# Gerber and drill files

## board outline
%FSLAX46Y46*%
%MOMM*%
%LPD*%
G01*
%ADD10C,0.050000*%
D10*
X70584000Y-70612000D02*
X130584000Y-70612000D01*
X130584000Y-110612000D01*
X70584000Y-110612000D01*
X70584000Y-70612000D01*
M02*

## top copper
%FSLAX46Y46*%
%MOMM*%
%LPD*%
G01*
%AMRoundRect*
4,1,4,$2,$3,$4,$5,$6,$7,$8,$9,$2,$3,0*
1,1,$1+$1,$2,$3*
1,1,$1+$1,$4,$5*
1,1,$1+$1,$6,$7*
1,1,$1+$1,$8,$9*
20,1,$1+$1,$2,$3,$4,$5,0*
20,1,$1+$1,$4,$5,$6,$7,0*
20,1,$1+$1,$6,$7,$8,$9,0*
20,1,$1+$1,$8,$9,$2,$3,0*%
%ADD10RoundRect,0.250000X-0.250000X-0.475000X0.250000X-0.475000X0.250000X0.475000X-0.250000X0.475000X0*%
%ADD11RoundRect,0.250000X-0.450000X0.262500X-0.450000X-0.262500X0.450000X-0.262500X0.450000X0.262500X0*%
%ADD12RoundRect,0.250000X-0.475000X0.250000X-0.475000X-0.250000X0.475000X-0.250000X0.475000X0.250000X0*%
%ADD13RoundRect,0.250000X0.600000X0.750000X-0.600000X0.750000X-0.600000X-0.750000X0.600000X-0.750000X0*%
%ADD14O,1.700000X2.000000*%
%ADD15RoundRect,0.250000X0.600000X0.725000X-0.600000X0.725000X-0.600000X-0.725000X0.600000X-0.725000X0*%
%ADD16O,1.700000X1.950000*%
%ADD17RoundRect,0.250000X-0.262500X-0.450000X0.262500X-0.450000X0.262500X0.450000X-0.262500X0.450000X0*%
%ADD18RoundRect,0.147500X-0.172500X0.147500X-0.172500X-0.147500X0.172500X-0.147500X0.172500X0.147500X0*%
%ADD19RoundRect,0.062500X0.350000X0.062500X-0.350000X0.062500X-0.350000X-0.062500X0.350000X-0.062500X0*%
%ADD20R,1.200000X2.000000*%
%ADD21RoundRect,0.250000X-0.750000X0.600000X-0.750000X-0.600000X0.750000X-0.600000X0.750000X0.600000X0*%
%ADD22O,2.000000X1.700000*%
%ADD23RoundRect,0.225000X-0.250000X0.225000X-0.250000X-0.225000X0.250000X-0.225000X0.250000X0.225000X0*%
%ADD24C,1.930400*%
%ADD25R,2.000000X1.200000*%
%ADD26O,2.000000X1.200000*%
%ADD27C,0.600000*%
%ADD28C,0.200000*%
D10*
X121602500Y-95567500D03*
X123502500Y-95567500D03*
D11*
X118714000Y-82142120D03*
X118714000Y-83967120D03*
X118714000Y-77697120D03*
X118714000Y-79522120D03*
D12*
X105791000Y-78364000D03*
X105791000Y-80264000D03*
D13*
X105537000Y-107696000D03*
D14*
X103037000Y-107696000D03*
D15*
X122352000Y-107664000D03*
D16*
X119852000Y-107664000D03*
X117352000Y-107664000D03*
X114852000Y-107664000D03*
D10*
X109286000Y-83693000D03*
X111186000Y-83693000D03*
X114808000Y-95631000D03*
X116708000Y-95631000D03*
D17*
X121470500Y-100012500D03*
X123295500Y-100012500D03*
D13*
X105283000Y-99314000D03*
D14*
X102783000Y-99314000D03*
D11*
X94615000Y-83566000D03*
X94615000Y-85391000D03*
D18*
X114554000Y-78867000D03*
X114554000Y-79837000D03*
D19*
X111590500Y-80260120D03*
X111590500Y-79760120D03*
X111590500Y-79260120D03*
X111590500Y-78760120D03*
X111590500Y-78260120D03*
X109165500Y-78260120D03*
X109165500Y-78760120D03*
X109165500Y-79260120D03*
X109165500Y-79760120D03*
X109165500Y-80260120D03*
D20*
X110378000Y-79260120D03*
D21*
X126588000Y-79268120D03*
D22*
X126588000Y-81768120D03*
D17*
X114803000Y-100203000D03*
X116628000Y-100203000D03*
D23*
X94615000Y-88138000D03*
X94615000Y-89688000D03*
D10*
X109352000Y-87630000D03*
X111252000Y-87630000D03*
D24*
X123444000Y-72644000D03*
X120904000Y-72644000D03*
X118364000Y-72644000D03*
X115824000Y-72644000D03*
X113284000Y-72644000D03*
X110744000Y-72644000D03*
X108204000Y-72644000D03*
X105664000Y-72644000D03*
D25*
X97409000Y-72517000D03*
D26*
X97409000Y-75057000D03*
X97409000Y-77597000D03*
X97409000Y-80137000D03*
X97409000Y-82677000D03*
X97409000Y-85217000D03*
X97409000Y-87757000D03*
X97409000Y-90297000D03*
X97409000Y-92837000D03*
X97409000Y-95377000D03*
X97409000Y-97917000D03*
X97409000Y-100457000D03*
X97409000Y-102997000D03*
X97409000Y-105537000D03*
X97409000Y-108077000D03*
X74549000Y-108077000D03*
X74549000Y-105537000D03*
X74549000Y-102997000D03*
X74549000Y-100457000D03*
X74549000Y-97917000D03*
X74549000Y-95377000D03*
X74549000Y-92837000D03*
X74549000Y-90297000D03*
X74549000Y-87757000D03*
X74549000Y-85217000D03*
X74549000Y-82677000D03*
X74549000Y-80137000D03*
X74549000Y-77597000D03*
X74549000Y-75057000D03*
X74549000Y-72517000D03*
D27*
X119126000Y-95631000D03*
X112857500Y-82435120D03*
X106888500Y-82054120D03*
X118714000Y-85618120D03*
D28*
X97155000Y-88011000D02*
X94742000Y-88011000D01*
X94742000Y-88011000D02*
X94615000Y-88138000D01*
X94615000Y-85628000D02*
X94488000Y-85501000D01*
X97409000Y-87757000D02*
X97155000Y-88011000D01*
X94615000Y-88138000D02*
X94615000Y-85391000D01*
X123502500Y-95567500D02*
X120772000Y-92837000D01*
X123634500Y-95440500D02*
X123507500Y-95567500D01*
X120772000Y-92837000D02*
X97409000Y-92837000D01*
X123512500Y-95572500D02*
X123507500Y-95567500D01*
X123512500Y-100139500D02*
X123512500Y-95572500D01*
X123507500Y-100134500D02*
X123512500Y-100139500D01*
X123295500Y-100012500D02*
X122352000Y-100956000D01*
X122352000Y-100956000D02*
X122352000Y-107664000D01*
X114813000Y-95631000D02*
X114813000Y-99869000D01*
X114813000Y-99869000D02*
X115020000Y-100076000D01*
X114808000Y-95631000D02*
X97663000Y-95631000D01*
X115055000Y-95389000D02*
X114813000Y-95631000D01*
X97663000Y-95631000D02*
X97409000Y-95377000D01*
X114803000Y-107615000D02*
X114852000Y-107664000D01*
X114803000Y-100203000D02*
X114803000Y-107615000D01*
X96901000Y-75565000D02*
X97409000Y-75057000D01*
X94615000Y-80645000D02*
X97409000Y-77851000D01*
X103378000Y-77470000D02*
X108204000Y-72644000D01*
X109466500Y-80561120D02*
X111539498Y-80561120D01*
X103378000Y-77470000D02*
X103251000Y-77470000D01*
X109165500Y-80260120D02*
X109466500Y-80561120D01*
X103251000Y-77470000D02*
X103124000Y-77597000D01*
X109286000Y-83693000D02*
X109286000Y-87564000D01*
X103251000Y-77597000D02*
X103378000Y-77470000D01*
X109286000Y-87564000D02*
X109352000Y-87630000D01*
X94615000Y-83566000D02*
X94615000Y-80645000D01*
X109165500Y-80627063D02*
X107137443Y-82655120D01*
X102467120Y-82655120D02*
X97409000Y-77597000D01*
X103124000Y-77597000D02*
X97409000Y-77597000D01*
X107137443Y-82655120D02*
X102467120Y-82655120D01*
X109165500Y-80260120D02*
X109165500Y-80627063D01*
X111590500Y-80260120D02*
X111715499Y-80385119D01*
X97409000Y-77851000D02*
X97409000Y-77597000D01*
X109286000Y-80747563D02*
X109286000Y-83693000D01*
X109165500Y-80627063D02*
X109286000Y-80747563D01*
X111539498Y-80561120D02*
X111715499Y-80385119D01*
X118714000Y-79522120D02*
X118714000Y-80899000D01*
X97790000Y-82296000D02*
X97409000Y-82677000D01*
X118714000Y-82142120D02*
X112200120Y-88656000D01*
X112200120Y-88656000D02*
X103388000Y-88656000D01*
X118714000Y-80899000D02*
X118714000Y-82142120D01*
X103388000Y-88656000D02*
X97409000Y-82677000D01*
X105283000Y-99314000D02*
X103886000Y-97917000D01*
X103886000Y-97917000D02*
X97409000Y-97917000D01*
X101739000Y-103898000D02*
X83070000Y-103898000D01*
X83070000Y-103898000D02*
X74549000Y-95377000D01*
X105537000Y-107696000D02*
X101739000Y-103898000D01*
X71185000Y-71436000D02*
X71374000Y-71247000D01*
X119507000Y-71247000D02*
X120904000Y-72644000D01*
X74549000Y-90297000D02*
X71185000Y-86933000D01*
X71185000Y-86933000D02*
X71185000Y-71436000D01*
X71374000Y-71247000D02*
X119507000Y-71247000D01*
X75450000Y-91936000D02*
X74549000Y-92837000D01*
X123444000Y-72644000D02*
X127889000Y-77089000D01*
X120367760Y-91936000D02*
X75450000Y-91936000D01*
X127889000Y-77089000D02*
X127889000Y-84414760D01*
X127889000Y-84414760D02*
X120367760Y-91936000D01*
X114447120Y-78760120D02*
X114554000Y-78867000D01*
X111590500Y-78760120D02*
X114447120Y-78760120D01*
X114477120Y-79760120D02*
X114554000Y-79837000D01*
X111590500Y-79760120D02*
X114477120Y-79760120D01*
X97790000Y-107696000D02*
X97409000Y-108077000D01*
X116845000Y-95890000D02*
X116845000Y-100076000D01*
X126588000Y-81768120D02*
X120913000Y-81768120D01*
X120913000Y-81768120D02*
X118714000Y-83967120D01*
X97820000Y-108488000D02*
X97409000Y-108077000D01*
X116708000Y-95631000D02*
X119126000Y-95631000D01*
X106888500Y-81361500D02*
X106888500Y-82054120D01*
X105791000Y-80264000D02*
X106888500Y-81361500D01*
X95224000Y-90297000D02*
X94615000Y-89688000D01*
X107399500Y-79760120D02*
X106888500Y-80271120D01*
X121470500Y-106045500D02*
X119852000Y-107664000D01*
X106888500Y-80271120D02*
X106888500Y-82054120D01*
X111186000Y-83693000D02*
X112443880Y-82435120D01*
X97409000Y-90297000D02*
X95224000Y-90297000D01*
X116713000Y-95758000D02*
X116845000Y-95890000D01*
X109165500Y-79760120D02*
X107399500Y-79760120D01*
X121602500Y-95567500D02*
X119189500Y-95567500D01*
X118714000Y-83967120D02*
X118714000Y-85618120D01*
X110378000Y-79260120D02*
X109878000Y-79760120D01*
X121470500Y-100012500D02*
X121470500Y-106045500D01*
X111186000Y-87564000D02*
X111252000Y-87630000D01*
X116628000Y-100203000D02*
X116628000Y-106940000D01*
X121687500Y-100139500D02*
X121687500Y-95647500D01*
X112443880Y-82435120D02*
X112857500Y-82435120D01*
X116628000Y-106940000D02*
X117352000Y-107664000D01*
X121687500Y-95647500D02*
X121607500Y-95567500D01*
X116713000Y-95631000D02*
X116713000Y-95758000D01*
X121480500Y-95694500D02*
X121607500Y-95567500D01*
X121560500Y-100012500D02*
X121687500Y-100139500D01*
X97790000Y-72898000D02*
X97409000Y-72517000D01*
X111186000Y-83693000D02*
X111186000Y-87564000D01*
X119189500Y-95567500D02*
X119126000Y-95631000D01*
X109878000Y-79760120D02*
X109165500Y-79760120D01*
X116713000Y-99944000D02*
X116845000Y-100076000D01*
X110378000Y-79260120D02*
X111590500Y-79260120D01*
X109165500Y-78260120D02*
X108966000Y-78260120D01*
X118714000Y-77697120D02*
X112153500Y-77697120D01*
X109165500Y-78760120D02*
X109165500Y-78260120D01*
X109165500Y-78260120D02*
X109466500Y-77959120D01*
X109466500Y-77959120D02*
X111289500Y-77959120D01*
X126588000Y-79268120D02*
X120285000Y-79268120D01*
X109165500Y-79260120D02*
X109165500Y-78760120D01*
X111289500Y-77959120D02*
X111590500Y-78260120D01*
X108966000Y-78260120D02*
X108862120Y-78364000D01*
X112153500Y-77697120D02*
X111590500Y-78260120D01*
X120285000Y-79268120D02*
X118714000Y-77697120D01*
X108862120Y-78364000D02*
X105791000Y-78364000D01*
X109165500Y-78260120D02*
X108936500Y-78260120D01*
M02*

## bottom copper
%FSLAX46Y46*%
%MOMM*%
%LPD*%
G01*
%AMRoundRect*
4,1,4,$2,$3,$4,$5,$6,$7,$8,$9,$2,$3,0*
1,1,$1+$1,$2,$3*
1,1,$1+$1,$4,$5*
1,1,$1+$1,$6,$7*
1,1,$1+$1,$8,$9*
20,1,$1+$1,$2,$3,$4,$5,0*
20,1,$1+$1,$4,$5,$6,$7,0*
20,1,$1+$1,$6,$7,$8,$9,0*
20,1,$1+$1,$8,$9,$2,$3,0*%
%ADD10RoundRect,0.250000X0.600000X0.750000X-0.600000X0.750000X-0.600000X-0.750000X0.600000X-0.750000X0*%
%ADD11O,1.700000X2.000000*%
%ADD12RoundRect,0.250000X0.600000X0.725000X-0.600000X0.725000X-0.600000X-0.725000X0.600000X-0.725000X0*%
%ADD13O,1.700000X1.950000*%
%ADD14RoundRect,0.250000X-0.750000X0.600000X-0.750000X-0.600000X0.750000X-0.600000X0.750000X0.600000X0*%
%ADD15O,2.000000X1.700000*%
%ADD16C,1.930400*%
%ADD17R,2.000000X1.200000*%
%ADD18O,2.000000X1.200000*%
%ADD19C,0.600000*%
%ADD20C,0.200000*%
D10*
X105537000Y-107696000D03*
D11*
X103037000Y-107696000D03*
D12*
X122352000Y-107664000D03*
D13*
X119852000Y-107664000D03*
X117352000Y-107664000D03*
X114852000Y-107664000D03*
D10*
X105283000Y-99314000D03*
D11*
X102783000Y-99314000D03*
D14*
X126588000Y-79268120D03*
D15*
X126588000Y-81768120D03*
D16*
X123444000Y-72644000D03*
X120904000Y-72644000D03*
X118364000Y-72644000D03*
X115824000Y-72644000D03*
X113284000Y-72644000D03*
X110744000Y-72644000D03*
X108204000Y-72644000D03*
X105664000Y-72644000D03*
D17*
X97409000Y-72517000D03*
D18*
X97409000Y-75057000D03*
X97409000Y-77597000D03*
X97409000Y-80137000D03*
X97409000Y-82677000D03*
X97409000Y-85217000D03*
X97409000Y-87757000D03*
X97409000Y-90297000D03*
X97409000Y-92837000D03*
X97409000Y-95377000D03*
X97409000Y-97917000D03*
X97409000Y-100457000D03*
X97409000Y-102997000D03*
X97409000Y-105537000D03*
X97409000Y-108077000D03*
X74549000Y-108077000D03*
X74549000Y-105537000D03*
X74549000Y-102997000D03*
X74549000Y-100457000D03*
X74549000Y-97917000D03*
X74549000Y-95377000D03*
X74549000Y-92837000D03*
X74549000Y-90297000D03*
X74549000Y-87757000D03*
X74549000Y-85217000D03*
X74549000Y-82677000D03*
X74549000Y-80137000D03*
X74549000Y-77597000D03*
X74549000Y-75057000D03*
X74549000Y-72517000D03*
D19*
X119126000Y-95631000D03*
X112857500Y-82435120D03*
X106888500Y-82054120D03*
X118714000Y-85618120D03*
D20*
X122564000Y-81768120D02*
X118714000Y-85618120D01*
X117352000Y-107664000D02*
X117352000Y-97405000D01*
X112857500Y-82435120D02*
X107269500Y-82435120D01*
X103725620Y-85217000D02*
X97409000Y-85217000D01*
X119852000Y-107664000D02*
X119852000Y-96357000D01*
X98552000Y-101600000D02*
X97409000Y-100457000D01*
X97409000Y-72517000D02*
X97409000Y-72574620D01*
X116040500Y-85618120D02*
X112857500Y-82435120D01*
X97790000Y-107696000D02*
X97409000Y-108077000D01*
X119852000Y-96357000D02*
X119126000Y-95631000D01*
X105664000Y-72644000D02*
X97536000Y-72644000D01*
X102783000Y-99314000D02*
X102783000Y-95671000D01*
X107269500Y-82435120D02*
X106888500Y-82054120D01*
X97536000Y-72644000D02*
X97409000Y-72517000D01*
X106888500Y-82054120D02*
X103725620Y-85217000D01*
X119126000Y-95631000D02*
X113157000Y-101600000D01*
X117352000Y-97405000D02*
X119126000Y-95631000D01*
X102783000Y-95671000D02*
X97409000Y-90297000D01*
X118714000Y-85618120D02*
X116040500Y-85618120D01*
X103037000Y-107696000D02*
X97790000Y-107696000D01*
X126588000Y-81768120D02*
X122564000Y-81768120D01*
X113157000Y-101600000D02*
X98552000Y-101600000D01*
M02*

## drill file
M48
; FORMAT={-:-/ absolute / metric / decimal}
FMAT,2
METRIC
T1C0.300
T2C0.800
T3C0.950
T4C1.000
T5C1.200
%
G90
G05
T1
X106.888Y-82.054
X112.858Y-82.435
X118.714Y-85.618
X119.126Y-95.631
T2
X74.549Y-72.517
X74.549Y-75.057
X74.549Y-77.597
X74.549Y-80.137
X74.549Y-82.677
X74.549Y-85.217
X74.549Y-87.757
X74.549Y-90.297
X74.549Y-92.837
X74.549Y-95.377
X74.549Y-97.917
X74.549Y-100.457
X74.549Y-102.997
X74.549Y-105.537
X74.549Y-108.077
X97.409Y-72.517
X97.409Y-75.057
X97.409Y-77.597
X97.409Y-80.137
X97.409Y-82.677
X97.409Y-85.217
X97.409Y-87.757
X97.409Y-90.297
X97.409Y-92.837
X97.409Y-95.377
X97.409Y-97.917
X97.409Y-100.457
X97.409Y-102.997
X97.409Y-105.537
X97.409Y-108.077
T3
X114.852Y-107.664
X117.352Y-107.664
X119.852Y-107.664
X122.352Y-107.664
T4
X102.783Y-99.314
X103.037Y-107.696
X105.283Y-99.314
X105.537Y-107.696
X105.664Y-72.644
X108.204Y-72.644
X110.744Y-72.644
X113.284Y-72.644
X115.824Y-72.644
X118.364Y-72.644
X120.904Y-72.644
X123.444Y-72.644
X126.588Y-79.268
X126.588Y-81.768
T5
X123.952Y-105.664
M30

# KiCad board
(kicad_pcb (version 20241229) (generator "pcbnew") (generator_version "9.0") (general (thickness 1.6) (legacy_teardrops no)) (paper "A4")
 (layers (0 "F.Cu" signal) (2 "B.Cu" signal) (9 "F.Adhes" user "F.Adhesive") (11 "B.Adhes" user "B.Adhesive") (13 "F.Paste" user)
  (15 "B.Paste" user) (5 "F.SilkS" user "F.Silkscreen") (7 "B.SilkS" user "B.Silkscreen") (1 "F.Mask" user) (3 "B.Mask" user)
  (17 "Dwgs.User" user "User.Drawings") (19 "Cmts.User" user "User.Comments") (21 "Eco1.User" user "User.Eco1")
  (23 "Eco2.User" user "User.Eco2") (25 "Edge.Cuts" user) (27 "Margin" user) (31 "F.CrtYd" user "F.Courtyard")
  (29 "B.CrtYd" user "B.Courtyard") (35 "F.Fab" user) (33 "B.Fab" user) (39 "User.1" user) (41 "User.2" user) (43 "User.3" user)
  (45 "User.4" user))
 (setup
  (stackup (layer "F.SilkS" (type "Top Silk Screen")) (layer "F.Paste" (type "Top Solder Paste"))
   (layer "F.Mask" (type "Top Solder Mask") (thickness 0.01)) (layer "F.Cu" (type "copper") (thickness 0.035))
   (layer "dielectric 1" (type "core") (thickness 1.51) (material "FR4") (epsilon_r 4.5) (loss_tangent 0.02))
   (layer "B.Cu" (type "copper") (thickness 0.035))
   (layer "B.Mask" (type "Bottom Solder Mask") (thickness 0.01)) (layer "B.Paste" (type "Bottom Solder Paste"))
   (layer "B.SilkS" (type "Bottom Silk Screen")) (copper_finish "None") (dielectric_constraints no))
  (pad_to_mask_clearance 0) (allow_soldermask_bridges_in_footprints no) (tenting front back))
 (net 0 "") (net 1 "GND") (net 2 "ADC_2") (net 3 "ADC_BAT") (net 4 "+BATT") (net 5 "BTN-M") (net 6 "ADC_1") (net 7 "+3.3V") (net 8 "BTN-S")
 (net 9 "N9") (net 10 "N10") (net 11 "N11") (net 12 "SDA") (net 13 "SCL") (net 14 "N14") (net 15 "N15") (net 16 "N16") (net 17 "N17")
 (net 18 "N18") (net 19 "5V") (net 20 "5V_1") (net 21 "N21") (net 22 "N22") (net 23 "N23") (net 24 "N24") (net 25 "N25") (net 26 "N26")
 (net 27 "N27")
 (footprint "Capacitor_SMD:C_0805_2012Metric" (layer "F.Cu") (at 122.5525 95.5675)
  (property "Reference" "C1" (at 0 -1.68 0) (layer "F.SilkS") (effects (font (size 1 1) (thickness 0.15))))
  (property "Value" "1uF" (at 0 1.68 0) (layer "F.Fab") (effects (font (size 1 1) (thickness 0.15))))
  (pad "1" smd roundrect (at -0.95 0) (size 1 1.45) (layers "F.Cu" "F.Mask" "F.Paste") (roundrect_rratio 0.25) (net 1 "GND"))
  (pad "2" smd roundrect (at 0.95 0) (size 1 1.45) (layers "F.Cu" "F.Mask" "F.Paste") (roundrect_rratio 0.25) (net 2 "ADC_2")))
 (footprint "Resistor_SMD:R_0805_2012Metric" (layer "F.Cu") (at 118.714 83.05462 -90)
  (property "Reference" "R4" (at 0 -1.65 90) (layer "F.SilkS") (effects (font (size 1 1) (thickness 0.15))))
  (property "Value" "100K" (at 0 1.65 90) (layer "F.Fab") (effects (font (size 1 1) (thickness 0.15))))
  (pad "1" smd roundrect (at -0.9125 0 270) (size 1.025 1.4) (layers "F.Cu" "F.Mask" "F.Paste") (roundrect_rratio 0.243902)
   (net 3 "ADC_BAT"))
  (pad "2" smd roundrect (at 0.9125 0 270) (size 1.025 1.4) (layers "F.Cu" "F.Mask" "F.Paste") (roundrect_rratio 0.243902) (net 1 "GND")))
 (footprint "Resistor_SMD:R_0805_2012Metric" (layer "F.Cu") (at 118.714 78.60962 -90)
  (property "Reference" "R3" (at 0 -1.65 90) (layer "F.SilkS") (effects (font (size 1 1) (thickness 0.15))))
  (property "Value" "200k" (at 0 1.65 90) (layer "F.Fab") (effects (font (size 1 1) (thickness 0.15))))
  (pad "1" smd roundrect (at -0.9125 0 270) (size 1.025 1.4) (layers "F.Cu" "F.Mask" "F.Paste") (roundrect_rratio 0.243902) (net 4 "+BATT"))
  (pad "2" smd roundrect (at 0.9125 0 270) (size 1.025 1.4) (layers "F.Cu" "F.Mask" "F.Paste") (roundrect_rratio 0.243902) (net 3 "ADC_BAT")))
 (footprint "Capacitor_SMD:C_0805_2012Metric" (layer "F.Cu") (at 105.791 79.314 -90)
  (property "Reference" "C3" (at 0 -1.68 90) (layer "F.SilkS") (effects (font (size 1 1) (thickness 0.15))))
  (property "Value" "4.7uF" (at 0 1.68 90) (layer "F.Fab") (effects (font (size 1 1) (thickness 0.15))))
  (pad "1" smd roundrect (at -0.95 0 270) (size 1 1.45) (layers "F.Cu" "F.Mask" "F.Paste") (roundrect_rratio 0.25) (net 4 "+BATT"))
  (pad "2" smd roundrect (at 0.95 0 270) (size 1 1.45) (layers "F.Cu" "F.Mask" "F.Paste") (roundrect_rratio 0.25) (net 1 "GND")))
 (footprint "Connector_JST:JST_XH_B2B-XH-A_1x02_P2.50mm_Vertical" (layer "F.Cu") (at 105.537 107.696 180)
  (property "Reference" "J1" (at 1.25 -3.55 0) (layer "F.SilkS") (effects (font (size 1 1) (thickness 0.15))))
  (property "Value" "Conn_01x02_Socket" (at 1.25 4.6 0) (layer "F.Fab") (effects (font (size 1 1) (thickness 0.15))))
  (pad "1" thru_hole roundrect (at 0 0 180) (size 1.7 2) (drill 1) (layers "*.Cu" "*.Mask") (remove_unused_layers no)
   (roundrect_rratio 0.147059) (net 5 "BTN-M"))
  (pad "2" thru_hole oval (at 2.5 0 180) (size 1.7 2) (drill 1) (layers "*.Cu" "*.Mask") (remove_unused_layers no) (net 1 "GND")))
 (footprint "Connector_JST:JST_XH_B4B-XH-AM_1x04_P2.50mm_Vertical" (layer "F.Cu") (at 122.352 107.664 180)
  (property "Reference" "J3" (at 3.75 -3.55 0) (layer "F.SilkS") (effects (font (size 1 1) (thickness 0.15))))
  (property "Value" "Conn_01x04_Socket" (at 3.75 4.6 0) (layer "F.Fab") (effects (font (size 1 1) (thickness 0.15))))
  (pad "" np_thru_hole circle (at -1.6 2 180) (size 1.2 1.2) (drill 1.2) (layers "*.Cu" "*.Mask"))
  (pad "1" thru_hole roundrect (at 0 0 180) (size 1.7 1.95) (drill 0.95) (layers "*.Cu" "*.Mask") (remove_unused_layers no)
   (roundrect_rratio 0.147059) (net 2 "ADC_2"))
  (pad "2" thru_hole oval (at 2.5 0 180) (size 1.7 1.95) (drill 0.95) (layers "*.Cu" "*.Mask") (remove_unused_layers no) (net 1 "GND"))
  (pad "3" thru_hole oval (at 5 0 180) (size 1.7 1.95) (drill 0.95) (layers "*.Cu" "*.Mask") (remove_unused_layers no) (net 1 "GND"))
  (pad "4" thru_hole oval (at 7.5 0 180) (size 1.7 1.95) (drill 0.95) (layers "*.Cu" "*.Mask") (remove_unused_layers no) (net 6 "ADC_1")))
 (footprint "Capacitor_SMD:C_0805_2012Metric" (layer "F.Cu") (at 110.236 83.693)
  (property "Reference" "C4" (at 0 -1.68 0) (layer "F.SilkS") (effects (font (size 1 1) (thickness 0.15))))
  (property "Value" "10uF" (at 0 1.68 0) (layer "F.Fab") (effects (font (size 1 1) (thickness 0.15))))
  (pad "1" smd roundrect (at -0.95 0) (size 1 1.45) (layers "F.Cu" "F.Mask" "F.Paste") (roundrect_rratio 0.25) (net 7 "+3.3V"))
  (pad "2" smd roundrect (at 0.95 0) (size 1 1.45) (layers "F.Cu" "F.Mask" "F.Paste") (roundrect_rratio 0.25) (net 1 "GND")))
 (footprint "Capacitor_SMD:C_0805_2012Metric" (layer "F.Cu") (at 115.758 95.631)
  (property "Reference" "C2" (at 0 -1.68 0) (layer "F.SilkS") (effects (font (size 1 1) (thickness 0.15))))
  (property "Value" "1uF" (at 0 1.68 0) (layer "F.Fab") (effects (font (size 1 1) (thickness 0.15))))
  (pad "1" smd roundrect (at -0.95 0) (size 1 1.45) (layers "F.Cu" "F.Mask" "F.Paste") (roundrect_rratio 0.25) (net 6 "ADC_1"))
  (pad "2" smd roundrect (at 0.95 0) (size 1 1.45) (layers "F.Cu" "F.Mask" "F.Paste") (roundrect_rratio 0.25) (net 1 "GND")))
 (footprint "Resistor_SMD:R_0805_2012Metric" (layer "F.Cu") (at 122.383 100.0125)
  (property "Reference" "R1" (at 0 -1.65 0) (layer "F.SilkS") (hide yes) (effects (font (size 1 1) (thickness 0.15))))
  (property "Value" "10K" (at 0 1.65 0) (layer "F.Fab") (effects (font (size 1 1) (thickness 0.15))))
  (pad "1" smd roundrect (at -0.9125 0) (size 1.025 1.4) (layers "F.Cu" "F.Mask" "F.Paste") (roundrect_rratio 0.243902) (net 1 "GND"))
  (pad "2" smd roundrect (at 0.9125 0) (size 1.025 1.4) (layers "F.Cu" "F.Mask" "F.Paste") (roundrect_rratio 0.243902) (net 2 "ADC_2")))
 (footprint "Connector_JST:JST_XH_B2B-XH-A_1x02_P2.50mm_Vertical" (layer "F.Cu") (at 105.283 99.314 180)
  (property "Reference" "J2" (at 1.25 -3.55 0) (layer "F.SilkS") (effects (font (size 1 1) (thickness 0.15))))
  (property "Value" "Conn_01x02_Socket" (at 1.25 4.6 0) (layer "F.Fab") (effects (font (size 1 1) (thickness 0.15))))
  (pad "1" thru_hole roundrect (at 0 0 180) (size 1.7 2) (drill 1) (layers "*.Cu" "*.Mask") (remove_unused_layers no)
   (roundrect_rratio 0.147059) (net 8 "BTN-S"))
  (pad "2" thru_hole oval (at 2.5 0 180) (size 1.7 2) (drill 1) (layers "*.Cu" "*.Mask") (remove_unused_layers no) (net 1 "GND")))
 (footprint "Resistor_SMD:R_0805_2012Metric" (layer "F.Cu") (at 94.615 84.4785 -90)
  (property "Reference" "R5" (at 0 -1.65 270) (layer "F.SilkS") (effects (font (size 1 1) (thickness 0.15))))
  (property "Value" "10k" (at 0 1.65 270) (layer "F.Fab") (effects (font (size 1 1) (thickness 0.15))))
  (pad "1" smd roundrect (at -0.9125 0 270) (size 1.025 1.4) (layers "F.Cu" "F.Mask" "F.Paste") (roundrect_rratio 0.243902) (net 7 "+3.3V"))
  (pad "2" smd roundrect (at 0.9125 0 270) (size 1.025 1.4) (layers "F.Cu" "F.Mask" "F.Paste") (roundrect_rratio 0.243902) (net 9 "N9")))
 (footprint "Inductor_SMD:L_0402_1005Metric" (layer "F.Cu") (at 114.554 79.352 -90)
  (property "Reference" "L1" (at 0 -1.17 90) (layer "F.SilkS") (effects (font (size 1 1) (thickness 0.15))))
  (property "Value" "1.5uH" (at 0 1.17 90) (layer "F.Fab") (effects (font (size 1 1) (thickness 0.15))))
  (pad "1" smd roundrect (at -0.485 0 270) (size 0.59 0.64) (layers "F.Cu" "F.Mask" "F.Paste") (roundrect_rratio 0.25) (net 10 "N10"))
  (pad "2" smd roundrect (at 0.485 0 270) (size 0.59 0.64) (layers "F.Cu" "F.Mask" "F.Paste") (roundrect_rratio 0.25) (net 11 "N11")))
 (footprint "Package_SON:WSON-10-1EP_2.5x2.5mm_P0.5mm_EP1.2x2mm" (layer "F.Cu") (at 110.378 79.26012 180)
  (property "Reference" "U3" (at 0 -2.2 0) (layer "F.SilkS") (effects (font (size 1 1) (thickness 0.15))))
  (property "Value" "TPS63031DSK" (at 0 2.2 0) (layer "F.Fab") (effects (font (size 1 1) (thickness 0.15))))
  (pad "" smd roundrect (at -0.3 -0.5 180) (size 0.48 0.81) (layers "F.Paste") (roundrect_rratio 0.25))
  (pad "" smd roundrect (at -0.3 0.5 180) (size 0.48 0.81) (layers "F.Paste") (roundrect_rratio 0.25))
  (pad "" smd roundrect (at 0.3 -0.5 180) (size 0.48 0.81) (layers "F.Paste") (roundrect_rratio 0.25))
  (pad "" smd roundrect (at 0.3 0.5 180) (size 0.48 0.81) (layers "F.Paste") (roundrect_rratio 0.25))
  (pad "1" smd roundrect (at -1.2125 -1 180) (size 0.825 0.25) (layers "F.Cu" "F.Mask" "F.Paste") (roundrect_rratio 0.25) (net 7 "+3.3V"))
  (pad "2" smd roundrect (at -1.2125 -0.5 180) (size 0.825 0.25) (layers "F.Cu" "F.Mask" "F.Paste") (roundrect_rratio 0.25) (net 11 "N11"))
  (pad "3" smd roundrect (at -1.2125 0 180) (size 0.825 0.25) (layers "F.Cu" "F.Mask" "F.Paste") (roundrect_rratio 0.25) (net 1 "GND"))
  (pad "4" smd roundrect (at -1.2125 0.5 180) (size 0.825 0.25) (layers "F.Cu" "F.Mask" "F.Paste") (roundrect_rratio 0.25) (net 10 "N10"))
  (pad "5" smd roundrect (at -1.2125 1 180) (size 0.825 0.25) (layers "F.Cu" "F.Mask" "F.Paste") (roundrect_rratio 0.25) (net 4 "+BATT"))
  (pad "6" smd roundrect (at 1.2125 1 180) (size 0.825 0.25) (layers "F.Cu" "F.Mask" "F.Paste") (roundrect_rratio 0.25) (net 4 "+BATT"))
  (pad "7" smd roundrect (at 1.2125 0.5 180) (size 0.825 0.25) (layers "F.Cu" "F.Mask" "F.Paste") (roundrect_rratio 0.25) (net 4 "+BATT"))
  (pad "8" smd roundrect (at 1.2125 0 180) (size 0.825 0.25) (layers "F.Cu" "F.Mask" "F.Paste") (roundrect_rratio 0.25) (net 4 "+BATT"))
  (pad "9" smd roundrect (at 1.2125 -0.5 180) (size 0.825 0.25) (layers "F.Cu" "F.Mask" "F.Paste") (roundrect_rratio 0.25) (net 1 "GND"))
  (pad "10" smd roundrect (at 1.2125 -1 180) (size 0.825 0.25) (layers "F.Cu" "F.Mask" "F.Paste") (roundrect_rratio 0.25) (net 7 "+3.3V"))
  (pad "11" smd rect (at 0 0 180) (size 1.2 2) (layers "F.Cu" "F.Mask") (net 1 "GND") (zone_connect 2)))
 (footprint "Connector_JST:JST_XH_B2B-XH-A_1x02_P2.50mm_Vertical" (layer "F.Cu") (at 126.588 79.26812 -90)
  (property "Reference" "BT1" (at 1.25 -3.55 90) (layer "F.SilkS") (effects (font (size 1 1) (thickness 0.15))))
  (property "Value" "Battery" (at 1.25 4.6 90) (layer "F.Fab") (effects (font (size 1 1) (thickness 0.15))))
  (pad "1" thru_hole roundrect (at 0 0 270) (size 1.7 2) (drill 1) (layers "*.Cu" "*.Mask") (remove_unused_layers no)
   (roundrect_rratio 0.147059) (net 4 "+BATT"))
  (pad "2" thru_hole oval (at 2.5 0 270) (size 1.7 2) (drill 1) (layers "*.Cu" "*.Mask") (remove_unused_layers no) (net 1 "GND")))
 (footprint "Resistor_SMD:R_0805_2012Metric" (layer "F.Cu") (at 115.7155 100.203)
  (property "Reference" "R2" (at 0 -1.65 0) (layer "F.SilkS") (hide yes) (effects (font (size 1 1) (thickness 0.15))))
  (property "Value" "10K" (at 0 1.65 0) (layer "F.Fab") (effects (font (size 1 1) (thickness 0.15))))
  (pad "1" smd roundrect (at -0.9125 0) (size 1.025 1.4) (layers "F.Cu" "F.Mask" "F.Paste") (roundrect_rratio 0.243902) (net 6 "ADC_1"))
  (pad "2" smd roundrect (at 0.9125 0) (size 1.025 1.4) (layers "F.Cu" "F.Mask" "F.Paste") (roundrect_rratio 0.243902) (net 1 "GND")))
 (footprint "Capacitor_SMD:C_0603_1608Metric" (layer "F.Cu") (at 94.615 88.913 -90)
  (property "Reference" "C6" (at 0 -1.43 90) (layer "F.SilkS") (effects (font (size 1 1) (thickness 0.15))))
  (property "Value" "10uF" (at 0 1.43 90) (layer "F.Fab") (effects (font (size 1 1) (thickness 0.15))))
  (pad "1" smd roundrect (at -0.775 0 270) (size 0.9 0.95) (layers "F.Cu" "F.Mask" "F.Paste") (roundrect_rratio 0.25) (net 9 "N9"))
  (pad "2" smd roundrect (at 0.775 0 270) (size 0.9 0.95) (layers "F.Cu" "F.Mask" "F.Paste") (roundrect_rratio 0.25) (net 1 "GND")))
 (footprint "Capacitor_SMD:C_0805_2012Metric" (layer "F.Cu") (at 110.302 87.63)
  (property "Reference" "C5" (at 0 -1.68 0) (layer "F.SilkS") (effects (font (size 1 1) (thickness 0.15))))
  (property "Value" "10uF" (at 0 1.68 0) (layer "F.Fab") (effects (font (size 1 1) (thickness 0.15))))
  (pad "1" smd roundrect (at -0.95 0) (size 1 1.45) (layers "F.Cu" "F.Mask" "F.Paste") (roundrect_rratio 0.25) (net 7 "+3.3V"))
  (pad "2" smd roundrect (at 0.95 0) (size 1 1.45) (layers "F.Cu" "F.Mask" "F.Paste") (roundrect_rratio 0.25) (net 1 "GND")))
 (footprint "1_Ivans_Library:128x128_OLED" (layer "B.Cu") (at 123.444 72.644 180)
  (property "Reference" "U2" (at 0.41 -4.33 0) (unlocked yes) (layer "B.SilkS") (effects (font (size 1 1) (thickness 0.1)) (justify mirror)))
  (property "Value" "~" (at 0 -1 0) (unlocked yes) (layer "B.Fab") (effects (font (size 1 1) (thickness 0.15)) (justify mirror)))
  (pad "1" thru_hole circle (at 0 0 90) (size 1.9304 1.9304) (drill 1) (layers "*.Cu" "*.Mask") (remove_unused_layers no) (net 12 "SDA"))
  (pad "2" thru_hole circle (at 2.54 0 90) (size 1.9304 1.9304) (drill 1) (layers "*.Cu" "*.Mask") (remove_unused_layers no) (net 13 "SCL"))
  (pad "3" thru_hole circle (at 5.08 0 90) (size 1.9304 1.9304) (drill 1) (layers "*.Cu" "*.Mask") (remove_unused_layers no) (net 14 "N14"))
  (pad "4" thru_hole circle (at 7.62 0 90) (size 1.9304 1.9304) (drill 1) (layers "*.Cu" "*.Mask") (remove_unused_layers no) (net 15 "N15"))
  (pad "5" thru_hole circle (at 10.16 0 90) (size 1.9304 1.9304) (drill 1) (layers "*.Cu" "*.Mask") (remove_unused_layers no) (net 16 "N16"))
  (pad "6" thru_hole circle (at 12.7 0 90) (size 1.9304 1.9304) (drill 1) (layers "*.Cu" "*.Mask") (remove_unused_layers no) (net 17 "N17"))
  (pad "7" thru_hole circle (at 15.24 0 90) (size 1.9304 1.9304) (drill 1) (layers "*.Cu" "*.Mask") (remove_unused_layers no)
   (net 7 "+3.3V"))
  (pad "8" thru_hole circle (at 17.78 0 90) (size 1.9304 1.9304) (drill 1) (layers "*.Cu" "*.Mask") (remove_unused_layers no) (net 1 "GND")))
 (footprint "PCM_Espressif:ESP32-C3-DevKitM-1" (layer "B.Cu") (at 97.409 72.517 180)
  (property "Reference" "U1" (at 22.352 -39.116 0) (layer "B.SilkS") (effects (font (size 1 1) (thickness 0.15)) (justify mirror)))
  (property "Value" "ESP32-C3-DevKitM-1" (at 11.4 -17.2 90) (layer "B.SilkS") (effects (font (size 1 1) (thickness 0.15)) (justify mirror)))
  (pad "1" thru_hole rect (at 0 0 270) (size 1.2 2) (drill 0.8) (layers "*.Cu" "*.Mask") (remove_unused_layers no) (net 1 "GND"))
  (pad "2" thru_hole oval (at 0 -2.54 270) (size 1.2 2) (drill 0.8) (layers "*.Cu" "*.Mask") (remove_unused_layers no) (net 7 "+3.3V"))
  (pad "3" thru_hole oval (at 0 -5.08 270) (size 1.2 2) (drill 0.8) (layers "*.Cu" "*.Mask") (remove_unused_layers no) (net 7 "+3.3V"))
  (pad "4" thru_hole oval (at 0 -7.62 270) (size 1.2 2) (drill 0.8) (layers "*.Cu" "*.Mask") (remove_unused_layers no) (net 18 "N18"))
  (pad "5" thru_hole oval (at 0 -10.16 270) (size 1.2 2) (drill 0.8) (layers "*.Cu" "*.Mask") (remove_unused_layers no) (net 3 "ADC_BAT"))
  (pad "6" thru_hole oval (at 0 -12.7 270) (size 1.2 2) (drill 0.8) (layers "*.Cu" "*.Mask") (remove_unused_layers no) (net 1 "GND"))
  (pad "7" thru_hole oval (at 0 -15.24 270) (size 1.2 2) (drill 0.8) (layers "*.Cu" "*.Mask") (remove_unused_layers no) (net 9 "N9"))
  (pad "8" thru_hole oval (at 0 -17.78 270) (size 1.2 2) (drill 0.8) (layers "*.Cu" "*.Mask") (remove_unused_layers no) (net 1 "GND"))
  (pad "9" thru_hole oval (at 0 -20.32 270) (size 1.2 2) (drill 0.8) (layers "*.Cu" "*.Mask") (remove_unused_layers no) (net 2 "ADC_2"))
  (pad "10" thru_hole oval (at 0 -22.86 270) (size 1.2 2) (drill 0.8) (layers "*.Cu" "*.Mask") (remove_unused_layers no) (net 6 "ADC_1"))
  (pad "11" thru_hole oval (at 0 -25.4 270) (size 1.2 2) (drill 0.8) (layers "*.Cu" "*.Mask") (remove_unused_layers no) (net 8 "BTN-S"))
  (pad "12" thru_hole oval (at 0 -27.94 270) (size 1.2 2) (drill 0.8) (layers "*.Cu" "*.Mask") (remove_unused_layers no) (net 1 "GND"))
  (pad "13" thru_hole oval (at 0 -30.48 270) (size 1.2 2) (drill 0.8) (layers "*.Cu" "*.Mask") (remove_unused_layers no) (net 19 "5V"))
  (pad "14" thru_hole oval (at 0 -33.02 270) (size 1.2 2) (drill 0.8) (layers "*.Cu" "*.Mask") (remove_unused_layers no) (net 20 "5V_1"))
  (pad "15" thru_hole oval (at 0 -35.56 270) (size 1.2 2) (drill 0.8) (layers "*.Cu" "*.Mask") (remove_unused_layers no) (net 1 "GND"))
  (pad "16" thru_hole oval (at 22.86 -35.56 270) (size 1.2 2) (drill 0.8) (layers "*.Cu" "*.Mask") (remove_unused_layers no) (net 1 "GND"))
  (pad "17" thru_hole oval (at 22.86 -33.02 270) (size 1.2 2) (drill 0.8) (layers "*.Cu" "*.Mask") (remove_unused_layers no) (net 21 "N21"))
  (pad "18" thru_hole oval (at 22.86 -30.48 270) (size 1.2 2) (drill 0.8) (layers "*.Cu" "*.Mask") (remove_unused_layers no) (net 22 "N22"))
  (pad "19" thru_hole oval (at 22.86 -27.94 270) (size 1.2 2) (drill 0.8) (layers "*.Cu" "*.Mask") (remove_unused_layers no) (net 1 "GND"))
  (pad "20" thru_hole oval (at 22.86 -25.4 270) (size 1.2 2) (drill 0.8) (layers "*.Cu" "*.Mask") (remove_unused_layers no) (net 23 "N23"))
  (pad "21" thru_hole oval (at 22.86 -22.86 270) (size 1.2 2) (drill 0.8) (layers "*.Cu" "*.Mask") (remove_unused_layers no) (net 5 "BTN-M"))
  (pad "22" thru_hole oval (at 22.86 -20.32 270) (size 1.2 2) (drill 0.8) (layers "*.Cu" "*.Mask") (remove_unused_layers no) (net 12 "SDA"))
  (pad "23" thru_hole oval (at 22.86 -17.78 270) (size 1.2 2) (drill 0.8) (layers "*.Cu" "*.Mask") (remove_unused_layers no) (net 13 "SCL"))
  (pad "24" thru_hole oval (at 22.86 -15.24 270) (size 1.2 2) (drill 0.8) (layers "*.Cu" "*.Mask") (remove_unused_layers no) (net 1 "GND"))
  (pad "25" thru_hole oval (at 22.86 -12.7 270) (size 1.2 2) (drill 0.8) (layers "*.Cu" "*.Mask") (remove_unused_layers no) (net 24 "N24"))
  (pad "26" thru_hole oval (at 22.86 -10.16 270) (size 1.2 2) (drill 0.8) (layers "*.Cu" "*.Mask") (remove_unused_layers no) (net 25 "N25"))
  (pad "27" thru_hole oval (at 22.86 -7.62 270) (size 1.2 2) (drill 0.8) (layers "*.Cu" "*.Mask") (remove_unused_layers no) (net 1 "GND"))
  (pad "28" thru_hole oval (at 22.86 -5.08 270) (size 1.2 2) (drill 0.8) (layers "*.Cu" "*.Mask") (remove_unused_layers no) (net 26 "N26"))
  (pad "29" thru_hole oval (at 22.86 -2.54 270) (size 1.2 2) (drill 0.8) (layers "*.Cu" "*.Mask") (remove_unused_layers no) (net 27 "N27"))
  (pad "30" thru_hole oval (at 22.86 0 270) (size 1.2 2) (drill 0.8) (layers "*.Cu" "*.Mask") (remove_unused_layers no) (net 1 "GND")))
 (gr_rect (start 70.584 70.612) (end 130.584 110.612) (stroke (width 0.05) (type solid)) (fill no) (layer "Edge.Cuts"))
 (segment (start 97.155 88.011) (end 94.742 88.011) (width 0.2) (layer "F.Cu") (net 9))
 (segment (start 94.742 88.011) (end 94.615 88.138) (width 0.2) (layer "F.Cu") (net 9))
 (segment (start 94.615 85.628) (end 94.488 85.501) (width 0.2) (layer "F.Cu") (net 9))
 (segment (start 97.409 87.757) (end 97.155 88.011) (width 0.2) (layer "F.Cu") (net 9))
 (segment (start 94.615 88.138) (end 94.615 85.391) (width 0.2) (layer "F.Cu") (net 9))
 (segment (start 123.5025 95.5675) (end 120.772 92.837) (width 0.2) (layer "F.Cu") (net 2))
 (segment (start 123.6345 95.4405) (end 123.5075 95.5675) (width 0.2) (layer "F.Cu") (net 2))
 (segment (start 120.772 92.837) (end 97.409 92.837) (width 0.2) (layer "F.Cu") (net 2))
 (segment (start 123.5125 95.5725) (end 123.5075 95.5675) (width 0.2) (layer "F.Cu") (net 2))
 (segment (start 123.5125 100.1395) (end 123.5125 95.5725) (width 0.2) (layer "F.Cu") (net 2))
 (segment (start 123.5075 100.1345) (end 123.5125 100.1395) (width 0.2) (layer "F.Cu") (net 2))
 (segment (start 123.2955 100.0125) (end 122.352 100.956) (width 0.2) (layer "F.Cu") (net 2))
 (segment (start 122.352 100.956) (end 122.352 107.664) (width 0.2) (layer "F.Cu") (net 2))
 (segment (start 114.813 95.631) (end 114.813 99.869) (width 0.2) (layer "F.Cu") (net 6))
 (segment (start 114.813 99.869) (end 115.02 100.076) (width 0.2) (layer "F.Cu") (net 6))
 (segment (start 114.808 95.631) (end 97.663 95.631) (width 0.2) (layer "F.Cu") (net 6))
 (segment (start 115.055 95.389) (end 114.813 95.631) (width 0.2) (layer "F.Cu") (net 6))
 (segment (start 97.663 95.631) (end 97.409 95.377) (width 0.2) (layer "F.Cu") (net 6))
 (segment (start 114.803 107.615) (end 114.852 107.664) (width 0.2) (layer "F.Cu") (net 6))
 (segment (start 114.803 100.203) (end 114.803 107.615) (width 0.2) (layer "F.Cu") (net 6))
 (segment (start 96.901 75.565) (end 97.409 75.057) (width 0.2) (layer "F.Cu") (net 7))
 (segment (start 94.615 80.645) (end 97.409 77.851) (width 0.2) (layer "F.Cu") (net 7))
 (segment (start 103.378 77.47) (end 108.204 72.644) (width 0.2) (layer "F.Cu") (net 7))
 (segment (start 109.4665 80.56112) (end 111.539498 80.56112) (width 0.2) (layer "F.Cu") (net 7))
 (segment (start 103.378 77.47) (end 103.251 77.47) (width 0.2) (layer "F.Cu") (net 7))
 (segment (start 109.1655 80.26012) (end 109.4665 80.56112) (width 0.2) (layer "F.Cu") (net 7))
 (segment (start 103.251 77.47) (end 103.124 77.597) (width 0.2) (layer "F.Cu") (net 7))
 (segment (start 109.286 83.693) (end 109.286 87.564) (width 0.2) (layer "F.Cu") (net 7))
 (segment (start 103.251 77.597) (end 103.378 77.47) (width 0.2) (layer "F.Cu") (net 7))
 (segment (start 109.286 87.564) (end 109.352 87.63) (width 0.2) (layer "F.Cu") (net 7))
 (segment (start 94.615 83.566) (end 94.615 80.645) (width 0.2) (layer "F.Cu") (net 7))
 (segment (start 109.1655 80.627063) (end 107.137443 82.65512) (width 0.2) (layer "F.Cu") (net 7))
 (segment (start 102.46712 82.65512) (end 97.409 77.597) (width 0.2) (layer "F.Cu") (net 7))
 (segment (start 103.124 77.597) (end 97.409 77.597) (width 0.2) (layer "F.Cu") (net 7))
 (segment (start 107.137443 82.65512) (end 102.46712 82.65512) (width 0.2) (layer "F.Cu") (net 7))
 (segment (start 109.1655 80.26012) (end 109.1655 80.627063) (width 0.2) (layer "F.Cu") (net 7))
 (segment (start 111.5905 80.26012) (end 111.715499 80.385119) (width 0.2) (layer "F.Cu") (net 7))
 (segment (start 97.409 77.851) (end 97.409 77.597) (width 0.2) (layer "F.Cu") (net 7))
 (segment (start 109.286 80.747563) (end 109.286 83.693) (width 0.2) (layer "F.Cu") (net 7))
 (segment (start 109.1655 80.627063) (end 109.286 80.747563) (width 0.2) (layer "F.Cu") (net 7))
 (segment (start 111.539498 80.56112) (end 111.715499 80.385119) (width 0.2) (layer "F.Cu") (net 7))
 (segment (start 118.714 79.52212) (end 118.714 80.899) (width 0.2) (layer "F.Cu") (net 3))
 (segment (start 97.79 82.296) (end 97.409 82.677) (width 0.2) (layer "F.Cu") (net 3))
 (segment (start 118.714 82.14212) (end 112.20012 88.656) (width 0.2) (layer "F.Cu") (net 3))
 (segment (start 112.20012 88.656) (end 103.388 88.656) (width 0.2) (layer "F.Cu") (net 3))
 (segment (start 118.714 80.899) (end 118.714 82.14212) (width 0.2) (layer "F.Cu") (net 3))
 (segment (start 103.388 88.656) (end 97.409 82.677) (width 0.2) (layer "F.Cu") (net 3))
 (segment (start 105.283 99.314) (end 103.886 97.917) (width 0.2) (layer "F.Cu") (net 8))
 (segment (start 103.886 97.917) (end 97.409 97.917) (width 0.2) (layer "F.Cu") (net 8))
 (segment (start 101.739 103.898) (end 83.07 103.898) (width 0.2) (layer "F.Cu") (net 5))
 (segment (start 83.07 103.898) (end 74.549 95.377) (width 0.2) (layer "F.Cu") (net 5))
 (segment (start 105.537 107.696) (end 101.739 103.898) (width 0.2) (layer "F.Cu") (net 5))
 (segment (start 71.185 71.436) (end 71.374 71.247) (width 0.2) (layer "F.Cu") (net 13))
 (segment (start 119.507 71.247) (end 120.904 72.644) (width 0.2) (layer "F.Cu") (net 13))
 (segment (start 74.549 90.297) (end 71.185 86.933) (width 0.2) (layer "F.Cu") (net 13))
 (segment (start 71.185 86.933) (end 71.185 71.436) (width 0.2) (layer "F.Cu") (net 13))
 (segment (start 71.374 71.247) (end 119.507 71.247) (width 0.2) (layer "F.Cu") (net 13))
 (segment (start 75.45 91.936) (end 74.549 92.837) (width 0.2) (layer "F.Cu") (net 12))
 (segment (start 123.444 72.644) (end 127.889 77.089) (width 0.2) (layer "F.Cu") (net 12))
 (segment (start 120.36776 91.936) (end 75.45 91.936) (width 0.2) (layer "F.Cu") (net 12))
 (segment (start 127.889 77.089) (end 127.889 84.41476) (width 0.2) (layer "F.Cu") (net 12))
 (segment (start 127.889 84.41476) (end 120.36776 91.936) (width 0.2) (layer "F.Cu") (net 12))
 (segment (start 114.44712 78.76012) (end 114.554 78.867) (width 0.2) (layer "F.Cu") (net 10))
 (segment (start 111.5905 78.76012) (end 114.44712 78.76012) (width 0.2) (layer "F.Cu") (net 10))
 (segment (start 114.47712 79.76012) (end 114.554 79.837) (width 0.2) (layer "F.Cu") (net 11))
 (segment (start 111.5905 79.76012) (end 114.47712 79.76012) (width 0.2) (layer "F.Cu") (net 11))
 (segment (start 97.79 107.696) (end 97.409 108.077) (width 0.2) (layer "F.Cu") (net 1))
 (segment (start 116.845 95.89) (end 116.845 100.076) (width 0.2) (layer "F.Cu") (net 1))
 (segment (start 126.588 81.76812) (end 120.913 81.76812) (width 0.2) (layer "F.Cu") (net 1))
 (segment (start 120.913 81.76812) (end 118.714 83.96712) (width 0.2) (layer "F.Cu") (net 1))
 (segment (start 97.82 108.488) (end 97.409 108.077) (width 0.2) (layer "F.Cu") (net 1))
 (segment (start 116.708 95.631) (end 119.126 95.631) (width 0.2) (layer "F.Cu") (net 1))
 (segment (start 106.8885 81.3615) (end 106.8885 82.05412) (width 0.2) (layer "F.Cu") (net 1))
 (segment (start 105.791 80.264) (end 106.8885 81.3615) (width 0.2) (layer "F.Cu") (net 1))
 (segment (start 95.224 90.297) (end 94.615 89.688) (width 0.2) (layer "F.Cu") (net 1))
 (segment (start 107.3995 79.76012) (end 106.8885 80.27112) (width 0.2) (layer "F.Cu") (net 1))
 (segment (start 121.4705 106.0455) (end 119.852 107.664) (width 0.2) (layer "F.Cu") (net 1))
 (segment (start 106.8885 80.27112) (end 106.8885 82.05412) (width 0.2) (layer "F.Cu") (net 1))
 (segment (start 111.186 83.693) (end 112.44388 82.43512) (width 0.2) (layer "F.Cu") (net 1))
 (segment (start 97.409 90.297) (end 95.224 90.297) (width 0.2) (layer "F.Cu") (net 1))
 (segment (start 116.713 95.758) (end 116.845 95.89) (width 0.2) (layer "F.Cu") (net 1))
 (segment (start 109.1655 79.76012) (end 107.3995 79.76012) (width 0.2) (layer "F.Cu") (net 1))
 (segment (start 121.6025 95.5675) (end 119.1895 95.5675) (width 0.2) (layer "F.Cu") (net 1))
 (segment (start 118.714 83.96712) (end 118.714 85.61812) (width 0.2) (layer "F.Cu") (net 1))
 (segment (start 110.378 79.26012) (end 109.878 79.76012) (width 0.2) (layer "F.Cu") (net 1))
 (segment (start 121.4705 100.0125) (end 121.4705 106.0455) (width 0.2) (layer "F.Cu") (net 1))
 (segment (start 111.186 87.564) (end 111.252 87.63) (width 0.2) (layer "F.Cu") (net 1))
 (segment (start 116.628 100.203) (end 116.628 106.94) (width 0.2) (layer "F.Cu") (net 1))
 (segment (start 121.6875 100.1395) (end 121.6875 95.6475) (width 0.2) (layer "F.Cu") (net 1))
 (segment (start 112.44388 82.43512) (end 112.8575 82.43512) (width 0.2) (layer "F.Cu") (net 1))
 (segment (start 116.628 106.94) (end 117.352 107.664) (width 0.2) (layer "F.Cu") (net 1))
 (segment (start 121.6875 95.6475) (end 121.6075 95.5675) (width 0.2) (layer "F.Cu") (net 1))
 (segment (start 116.713 95.631) (end 116.713 95.758) (width 0.2) (layer "F.Cu") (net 1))
 (segment (start 121.4805 95.6945) (end 121.6075 95.5675) (width 0.2) (layer "F.Cu") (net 1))
 (segment (start 121.5605 100.0125) (end 121.6875 100.1395) (width 0.2) (layer "F.Cu") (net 1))
 (segment (start 97.79 72.898) (end 97.409 72.517) (width 0.2) (layer "F.Cu") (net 1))
 (segment (start 111.186 83.693) (end 111.186 87.564) (width 0.2) (layer "F.Cu") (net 1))
 (segment (start 119.1895 95.5675) (end 119.126 95.631) (width 0.2) (layer "F.Cu") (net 1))
 (segment (start 109.878 79.76012) (end 109.1655 79.76012) (width 0.2) (layer "F.Cu") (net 1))
 (segment (start 116.713 99.944) (end 116.845 100.076) (width 0.2) (layer "F.Cu") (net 1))
 (segment (start 110.378 79.26012) (end 111.5905 79.26012) (width 0.2) (layer "F.Cu") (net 1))
 (via (at 119.126 95.631) (size 0.6) (drill 0.3) (layers "F.Cu" "B.Cu") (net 1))
 (via (at 112.8575 82.43512) (size 0.6) (drill 0.3) (layers "F.Cu" "B.Cu") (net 1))
 (via (at 106.8885 82.05412) (size 0.6) (drill 0.3) (layers "F.Cu" "B.Cu") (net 1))
 (via (at 118.714 85.61812) (size 0.6) (drill 0.3) (layers "F.Cu" "B.Cu") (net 1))
 (segment (start 122.564 81.76812) (end 118.714 85.61812) (width 0.2) (layer "B.Cu") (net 1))
 (segment (start 117.352 107.664) (end 117.352 97.405) (width 0.2) (layer "B.Cu") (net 1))
 (segment (start 112.8575 82.43512) (end 107.2695 82.43512) (width 0.2) (layer "B.Cu") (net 1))
 (segment (start 103.72562 85.217) (end 97.409 85.217) (width 0.2) (layer "B.Cu") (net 1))
 (segment (start 119.852 107.664) (end 119.852 96.357) (width 0.2) (layer "B.Cu") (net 1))
 (segment (start 98.552 101.6) (end 97.409 100.457) (width 0.2) (layer "B.Cu") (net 1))
 (segment (start 97.409 72.517) (end 97.409 72.57462) (width 0.2) (layer "B.Cu") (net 1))
 (segment (start 116.0405 85.61812) (end 112.8575 82.43512) (width 0.2) (layer "B.Cu") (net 1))
 (segment (start 97.79 107.696) (end 97.409 108.077) (width 0.2) (layer "B.Cu") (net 1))
 (segment (start 119.852 96.357) (end 119.126 95.631) (width 0.2) (layer "B.Cu") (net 1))
 (segment (start 105.664 72.644) (end 97.536 72.644) (width 0.2) (layer "B.Cu") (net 1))
 (segment (start 102.783 99.314) (end 102.783 95.671) (width 0.2) (layer "B.Cu") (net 1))
 (segment (start 107.2695 82.43512) (end 106.8885 82.05412) (width 0.2) (layer "B.Cu") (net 1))
 (segment (start 97.536 72.644) (end 97.409 72.517) (width 0.2) (layer "B.Cu") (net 1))
 (segment (start 106.8885 82.05412) (end 103.72562 85.217) (width 0.2) (layer "B.Cu") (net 1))
 (segment (start 119.126 95.631) (end 113.157 101.6) (width 0.2) (layer "B.Cu") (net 1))
 (segment (start 117.352 97.405) (end 119.126 95.631) (width 0.2) (layer "B.Cu") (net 1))
 (segment (start 102.783 95.671) (end 97.409 90.297) (width 0.2) (layer "B.Cu") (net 1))
 (segment (start 118.714 85.61812) (end 116.0405 85.61812) (width 0.2) (layer "B.Cu") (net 1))
 (segment (start 103.037 107.696) (end 97.79 107.696) (width 0.2) (layer "B.Cu") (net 1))
 (segment (start 126.588 81.76812) (end 122.564 81.76812) (width 0.2) (layer "B.Cu") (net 1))
 (segment (start 113.157 101.6) (end 98.552 101.6) (width 0.2) (layer "B.Cu") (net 1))
 (segment (start 109.1655 78.26012) (end 108.966 78.26012) (width 0.2) (layer "F.Cu") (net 4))
 (segment (start 118.714 77.69712) (end 112.1535 77.69712) (width 0.2) (layer "F.Cu") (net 4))
 (segment (start 109.1655 78.76012) (end 109.1655 78.26012) (width 0.2) (layer "F.Cu") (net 4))
 (segment (start 109.1655 78.26012) (end 109.4665 77.95912) (width 0.2) (layer "F.Cu") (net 4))
 (segment (start 109.4665 77.95912) (end 111.2895 77.95912) (width 0.2) (layer "F.Cu") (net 4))
 (segment (start 126.588 79.26812) (end 120.285 79.26812) (width 0.2) (layer "F.Cu") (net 4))
 (segment (start 109.1655 79.26012) (end 109.1655 78.76012) (width 0.2) (layer "F.Cu") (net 4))
 (segment (start 111.2895 77.95912) (end 111.5905 78.26012) (width 0.2) (layer "F.Cu") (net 4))
 (segment (start 108.966 78.26012) (end 108.86212 78.364) (width 0.2) (layer "F.Cu") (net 4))
 (segment (start 112.1535 77.69712) (end 111.5905 78.26012) (width 0.2) (layer "F.Cu") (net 4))
 (segment (start 120.285 79.26812) (end 118.714 77.69712) (width 0.2) (layer "F.Cu") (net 4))
 (segment (start 108.86212 78.364) (end 105.791 78.364) (width 0.2) (layer "F.Cu") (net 4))
 (segment (start 109.1655 78.26012) (end 108.9365 78.26012) (width 0.2) (layer "F.Cu") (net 4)))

